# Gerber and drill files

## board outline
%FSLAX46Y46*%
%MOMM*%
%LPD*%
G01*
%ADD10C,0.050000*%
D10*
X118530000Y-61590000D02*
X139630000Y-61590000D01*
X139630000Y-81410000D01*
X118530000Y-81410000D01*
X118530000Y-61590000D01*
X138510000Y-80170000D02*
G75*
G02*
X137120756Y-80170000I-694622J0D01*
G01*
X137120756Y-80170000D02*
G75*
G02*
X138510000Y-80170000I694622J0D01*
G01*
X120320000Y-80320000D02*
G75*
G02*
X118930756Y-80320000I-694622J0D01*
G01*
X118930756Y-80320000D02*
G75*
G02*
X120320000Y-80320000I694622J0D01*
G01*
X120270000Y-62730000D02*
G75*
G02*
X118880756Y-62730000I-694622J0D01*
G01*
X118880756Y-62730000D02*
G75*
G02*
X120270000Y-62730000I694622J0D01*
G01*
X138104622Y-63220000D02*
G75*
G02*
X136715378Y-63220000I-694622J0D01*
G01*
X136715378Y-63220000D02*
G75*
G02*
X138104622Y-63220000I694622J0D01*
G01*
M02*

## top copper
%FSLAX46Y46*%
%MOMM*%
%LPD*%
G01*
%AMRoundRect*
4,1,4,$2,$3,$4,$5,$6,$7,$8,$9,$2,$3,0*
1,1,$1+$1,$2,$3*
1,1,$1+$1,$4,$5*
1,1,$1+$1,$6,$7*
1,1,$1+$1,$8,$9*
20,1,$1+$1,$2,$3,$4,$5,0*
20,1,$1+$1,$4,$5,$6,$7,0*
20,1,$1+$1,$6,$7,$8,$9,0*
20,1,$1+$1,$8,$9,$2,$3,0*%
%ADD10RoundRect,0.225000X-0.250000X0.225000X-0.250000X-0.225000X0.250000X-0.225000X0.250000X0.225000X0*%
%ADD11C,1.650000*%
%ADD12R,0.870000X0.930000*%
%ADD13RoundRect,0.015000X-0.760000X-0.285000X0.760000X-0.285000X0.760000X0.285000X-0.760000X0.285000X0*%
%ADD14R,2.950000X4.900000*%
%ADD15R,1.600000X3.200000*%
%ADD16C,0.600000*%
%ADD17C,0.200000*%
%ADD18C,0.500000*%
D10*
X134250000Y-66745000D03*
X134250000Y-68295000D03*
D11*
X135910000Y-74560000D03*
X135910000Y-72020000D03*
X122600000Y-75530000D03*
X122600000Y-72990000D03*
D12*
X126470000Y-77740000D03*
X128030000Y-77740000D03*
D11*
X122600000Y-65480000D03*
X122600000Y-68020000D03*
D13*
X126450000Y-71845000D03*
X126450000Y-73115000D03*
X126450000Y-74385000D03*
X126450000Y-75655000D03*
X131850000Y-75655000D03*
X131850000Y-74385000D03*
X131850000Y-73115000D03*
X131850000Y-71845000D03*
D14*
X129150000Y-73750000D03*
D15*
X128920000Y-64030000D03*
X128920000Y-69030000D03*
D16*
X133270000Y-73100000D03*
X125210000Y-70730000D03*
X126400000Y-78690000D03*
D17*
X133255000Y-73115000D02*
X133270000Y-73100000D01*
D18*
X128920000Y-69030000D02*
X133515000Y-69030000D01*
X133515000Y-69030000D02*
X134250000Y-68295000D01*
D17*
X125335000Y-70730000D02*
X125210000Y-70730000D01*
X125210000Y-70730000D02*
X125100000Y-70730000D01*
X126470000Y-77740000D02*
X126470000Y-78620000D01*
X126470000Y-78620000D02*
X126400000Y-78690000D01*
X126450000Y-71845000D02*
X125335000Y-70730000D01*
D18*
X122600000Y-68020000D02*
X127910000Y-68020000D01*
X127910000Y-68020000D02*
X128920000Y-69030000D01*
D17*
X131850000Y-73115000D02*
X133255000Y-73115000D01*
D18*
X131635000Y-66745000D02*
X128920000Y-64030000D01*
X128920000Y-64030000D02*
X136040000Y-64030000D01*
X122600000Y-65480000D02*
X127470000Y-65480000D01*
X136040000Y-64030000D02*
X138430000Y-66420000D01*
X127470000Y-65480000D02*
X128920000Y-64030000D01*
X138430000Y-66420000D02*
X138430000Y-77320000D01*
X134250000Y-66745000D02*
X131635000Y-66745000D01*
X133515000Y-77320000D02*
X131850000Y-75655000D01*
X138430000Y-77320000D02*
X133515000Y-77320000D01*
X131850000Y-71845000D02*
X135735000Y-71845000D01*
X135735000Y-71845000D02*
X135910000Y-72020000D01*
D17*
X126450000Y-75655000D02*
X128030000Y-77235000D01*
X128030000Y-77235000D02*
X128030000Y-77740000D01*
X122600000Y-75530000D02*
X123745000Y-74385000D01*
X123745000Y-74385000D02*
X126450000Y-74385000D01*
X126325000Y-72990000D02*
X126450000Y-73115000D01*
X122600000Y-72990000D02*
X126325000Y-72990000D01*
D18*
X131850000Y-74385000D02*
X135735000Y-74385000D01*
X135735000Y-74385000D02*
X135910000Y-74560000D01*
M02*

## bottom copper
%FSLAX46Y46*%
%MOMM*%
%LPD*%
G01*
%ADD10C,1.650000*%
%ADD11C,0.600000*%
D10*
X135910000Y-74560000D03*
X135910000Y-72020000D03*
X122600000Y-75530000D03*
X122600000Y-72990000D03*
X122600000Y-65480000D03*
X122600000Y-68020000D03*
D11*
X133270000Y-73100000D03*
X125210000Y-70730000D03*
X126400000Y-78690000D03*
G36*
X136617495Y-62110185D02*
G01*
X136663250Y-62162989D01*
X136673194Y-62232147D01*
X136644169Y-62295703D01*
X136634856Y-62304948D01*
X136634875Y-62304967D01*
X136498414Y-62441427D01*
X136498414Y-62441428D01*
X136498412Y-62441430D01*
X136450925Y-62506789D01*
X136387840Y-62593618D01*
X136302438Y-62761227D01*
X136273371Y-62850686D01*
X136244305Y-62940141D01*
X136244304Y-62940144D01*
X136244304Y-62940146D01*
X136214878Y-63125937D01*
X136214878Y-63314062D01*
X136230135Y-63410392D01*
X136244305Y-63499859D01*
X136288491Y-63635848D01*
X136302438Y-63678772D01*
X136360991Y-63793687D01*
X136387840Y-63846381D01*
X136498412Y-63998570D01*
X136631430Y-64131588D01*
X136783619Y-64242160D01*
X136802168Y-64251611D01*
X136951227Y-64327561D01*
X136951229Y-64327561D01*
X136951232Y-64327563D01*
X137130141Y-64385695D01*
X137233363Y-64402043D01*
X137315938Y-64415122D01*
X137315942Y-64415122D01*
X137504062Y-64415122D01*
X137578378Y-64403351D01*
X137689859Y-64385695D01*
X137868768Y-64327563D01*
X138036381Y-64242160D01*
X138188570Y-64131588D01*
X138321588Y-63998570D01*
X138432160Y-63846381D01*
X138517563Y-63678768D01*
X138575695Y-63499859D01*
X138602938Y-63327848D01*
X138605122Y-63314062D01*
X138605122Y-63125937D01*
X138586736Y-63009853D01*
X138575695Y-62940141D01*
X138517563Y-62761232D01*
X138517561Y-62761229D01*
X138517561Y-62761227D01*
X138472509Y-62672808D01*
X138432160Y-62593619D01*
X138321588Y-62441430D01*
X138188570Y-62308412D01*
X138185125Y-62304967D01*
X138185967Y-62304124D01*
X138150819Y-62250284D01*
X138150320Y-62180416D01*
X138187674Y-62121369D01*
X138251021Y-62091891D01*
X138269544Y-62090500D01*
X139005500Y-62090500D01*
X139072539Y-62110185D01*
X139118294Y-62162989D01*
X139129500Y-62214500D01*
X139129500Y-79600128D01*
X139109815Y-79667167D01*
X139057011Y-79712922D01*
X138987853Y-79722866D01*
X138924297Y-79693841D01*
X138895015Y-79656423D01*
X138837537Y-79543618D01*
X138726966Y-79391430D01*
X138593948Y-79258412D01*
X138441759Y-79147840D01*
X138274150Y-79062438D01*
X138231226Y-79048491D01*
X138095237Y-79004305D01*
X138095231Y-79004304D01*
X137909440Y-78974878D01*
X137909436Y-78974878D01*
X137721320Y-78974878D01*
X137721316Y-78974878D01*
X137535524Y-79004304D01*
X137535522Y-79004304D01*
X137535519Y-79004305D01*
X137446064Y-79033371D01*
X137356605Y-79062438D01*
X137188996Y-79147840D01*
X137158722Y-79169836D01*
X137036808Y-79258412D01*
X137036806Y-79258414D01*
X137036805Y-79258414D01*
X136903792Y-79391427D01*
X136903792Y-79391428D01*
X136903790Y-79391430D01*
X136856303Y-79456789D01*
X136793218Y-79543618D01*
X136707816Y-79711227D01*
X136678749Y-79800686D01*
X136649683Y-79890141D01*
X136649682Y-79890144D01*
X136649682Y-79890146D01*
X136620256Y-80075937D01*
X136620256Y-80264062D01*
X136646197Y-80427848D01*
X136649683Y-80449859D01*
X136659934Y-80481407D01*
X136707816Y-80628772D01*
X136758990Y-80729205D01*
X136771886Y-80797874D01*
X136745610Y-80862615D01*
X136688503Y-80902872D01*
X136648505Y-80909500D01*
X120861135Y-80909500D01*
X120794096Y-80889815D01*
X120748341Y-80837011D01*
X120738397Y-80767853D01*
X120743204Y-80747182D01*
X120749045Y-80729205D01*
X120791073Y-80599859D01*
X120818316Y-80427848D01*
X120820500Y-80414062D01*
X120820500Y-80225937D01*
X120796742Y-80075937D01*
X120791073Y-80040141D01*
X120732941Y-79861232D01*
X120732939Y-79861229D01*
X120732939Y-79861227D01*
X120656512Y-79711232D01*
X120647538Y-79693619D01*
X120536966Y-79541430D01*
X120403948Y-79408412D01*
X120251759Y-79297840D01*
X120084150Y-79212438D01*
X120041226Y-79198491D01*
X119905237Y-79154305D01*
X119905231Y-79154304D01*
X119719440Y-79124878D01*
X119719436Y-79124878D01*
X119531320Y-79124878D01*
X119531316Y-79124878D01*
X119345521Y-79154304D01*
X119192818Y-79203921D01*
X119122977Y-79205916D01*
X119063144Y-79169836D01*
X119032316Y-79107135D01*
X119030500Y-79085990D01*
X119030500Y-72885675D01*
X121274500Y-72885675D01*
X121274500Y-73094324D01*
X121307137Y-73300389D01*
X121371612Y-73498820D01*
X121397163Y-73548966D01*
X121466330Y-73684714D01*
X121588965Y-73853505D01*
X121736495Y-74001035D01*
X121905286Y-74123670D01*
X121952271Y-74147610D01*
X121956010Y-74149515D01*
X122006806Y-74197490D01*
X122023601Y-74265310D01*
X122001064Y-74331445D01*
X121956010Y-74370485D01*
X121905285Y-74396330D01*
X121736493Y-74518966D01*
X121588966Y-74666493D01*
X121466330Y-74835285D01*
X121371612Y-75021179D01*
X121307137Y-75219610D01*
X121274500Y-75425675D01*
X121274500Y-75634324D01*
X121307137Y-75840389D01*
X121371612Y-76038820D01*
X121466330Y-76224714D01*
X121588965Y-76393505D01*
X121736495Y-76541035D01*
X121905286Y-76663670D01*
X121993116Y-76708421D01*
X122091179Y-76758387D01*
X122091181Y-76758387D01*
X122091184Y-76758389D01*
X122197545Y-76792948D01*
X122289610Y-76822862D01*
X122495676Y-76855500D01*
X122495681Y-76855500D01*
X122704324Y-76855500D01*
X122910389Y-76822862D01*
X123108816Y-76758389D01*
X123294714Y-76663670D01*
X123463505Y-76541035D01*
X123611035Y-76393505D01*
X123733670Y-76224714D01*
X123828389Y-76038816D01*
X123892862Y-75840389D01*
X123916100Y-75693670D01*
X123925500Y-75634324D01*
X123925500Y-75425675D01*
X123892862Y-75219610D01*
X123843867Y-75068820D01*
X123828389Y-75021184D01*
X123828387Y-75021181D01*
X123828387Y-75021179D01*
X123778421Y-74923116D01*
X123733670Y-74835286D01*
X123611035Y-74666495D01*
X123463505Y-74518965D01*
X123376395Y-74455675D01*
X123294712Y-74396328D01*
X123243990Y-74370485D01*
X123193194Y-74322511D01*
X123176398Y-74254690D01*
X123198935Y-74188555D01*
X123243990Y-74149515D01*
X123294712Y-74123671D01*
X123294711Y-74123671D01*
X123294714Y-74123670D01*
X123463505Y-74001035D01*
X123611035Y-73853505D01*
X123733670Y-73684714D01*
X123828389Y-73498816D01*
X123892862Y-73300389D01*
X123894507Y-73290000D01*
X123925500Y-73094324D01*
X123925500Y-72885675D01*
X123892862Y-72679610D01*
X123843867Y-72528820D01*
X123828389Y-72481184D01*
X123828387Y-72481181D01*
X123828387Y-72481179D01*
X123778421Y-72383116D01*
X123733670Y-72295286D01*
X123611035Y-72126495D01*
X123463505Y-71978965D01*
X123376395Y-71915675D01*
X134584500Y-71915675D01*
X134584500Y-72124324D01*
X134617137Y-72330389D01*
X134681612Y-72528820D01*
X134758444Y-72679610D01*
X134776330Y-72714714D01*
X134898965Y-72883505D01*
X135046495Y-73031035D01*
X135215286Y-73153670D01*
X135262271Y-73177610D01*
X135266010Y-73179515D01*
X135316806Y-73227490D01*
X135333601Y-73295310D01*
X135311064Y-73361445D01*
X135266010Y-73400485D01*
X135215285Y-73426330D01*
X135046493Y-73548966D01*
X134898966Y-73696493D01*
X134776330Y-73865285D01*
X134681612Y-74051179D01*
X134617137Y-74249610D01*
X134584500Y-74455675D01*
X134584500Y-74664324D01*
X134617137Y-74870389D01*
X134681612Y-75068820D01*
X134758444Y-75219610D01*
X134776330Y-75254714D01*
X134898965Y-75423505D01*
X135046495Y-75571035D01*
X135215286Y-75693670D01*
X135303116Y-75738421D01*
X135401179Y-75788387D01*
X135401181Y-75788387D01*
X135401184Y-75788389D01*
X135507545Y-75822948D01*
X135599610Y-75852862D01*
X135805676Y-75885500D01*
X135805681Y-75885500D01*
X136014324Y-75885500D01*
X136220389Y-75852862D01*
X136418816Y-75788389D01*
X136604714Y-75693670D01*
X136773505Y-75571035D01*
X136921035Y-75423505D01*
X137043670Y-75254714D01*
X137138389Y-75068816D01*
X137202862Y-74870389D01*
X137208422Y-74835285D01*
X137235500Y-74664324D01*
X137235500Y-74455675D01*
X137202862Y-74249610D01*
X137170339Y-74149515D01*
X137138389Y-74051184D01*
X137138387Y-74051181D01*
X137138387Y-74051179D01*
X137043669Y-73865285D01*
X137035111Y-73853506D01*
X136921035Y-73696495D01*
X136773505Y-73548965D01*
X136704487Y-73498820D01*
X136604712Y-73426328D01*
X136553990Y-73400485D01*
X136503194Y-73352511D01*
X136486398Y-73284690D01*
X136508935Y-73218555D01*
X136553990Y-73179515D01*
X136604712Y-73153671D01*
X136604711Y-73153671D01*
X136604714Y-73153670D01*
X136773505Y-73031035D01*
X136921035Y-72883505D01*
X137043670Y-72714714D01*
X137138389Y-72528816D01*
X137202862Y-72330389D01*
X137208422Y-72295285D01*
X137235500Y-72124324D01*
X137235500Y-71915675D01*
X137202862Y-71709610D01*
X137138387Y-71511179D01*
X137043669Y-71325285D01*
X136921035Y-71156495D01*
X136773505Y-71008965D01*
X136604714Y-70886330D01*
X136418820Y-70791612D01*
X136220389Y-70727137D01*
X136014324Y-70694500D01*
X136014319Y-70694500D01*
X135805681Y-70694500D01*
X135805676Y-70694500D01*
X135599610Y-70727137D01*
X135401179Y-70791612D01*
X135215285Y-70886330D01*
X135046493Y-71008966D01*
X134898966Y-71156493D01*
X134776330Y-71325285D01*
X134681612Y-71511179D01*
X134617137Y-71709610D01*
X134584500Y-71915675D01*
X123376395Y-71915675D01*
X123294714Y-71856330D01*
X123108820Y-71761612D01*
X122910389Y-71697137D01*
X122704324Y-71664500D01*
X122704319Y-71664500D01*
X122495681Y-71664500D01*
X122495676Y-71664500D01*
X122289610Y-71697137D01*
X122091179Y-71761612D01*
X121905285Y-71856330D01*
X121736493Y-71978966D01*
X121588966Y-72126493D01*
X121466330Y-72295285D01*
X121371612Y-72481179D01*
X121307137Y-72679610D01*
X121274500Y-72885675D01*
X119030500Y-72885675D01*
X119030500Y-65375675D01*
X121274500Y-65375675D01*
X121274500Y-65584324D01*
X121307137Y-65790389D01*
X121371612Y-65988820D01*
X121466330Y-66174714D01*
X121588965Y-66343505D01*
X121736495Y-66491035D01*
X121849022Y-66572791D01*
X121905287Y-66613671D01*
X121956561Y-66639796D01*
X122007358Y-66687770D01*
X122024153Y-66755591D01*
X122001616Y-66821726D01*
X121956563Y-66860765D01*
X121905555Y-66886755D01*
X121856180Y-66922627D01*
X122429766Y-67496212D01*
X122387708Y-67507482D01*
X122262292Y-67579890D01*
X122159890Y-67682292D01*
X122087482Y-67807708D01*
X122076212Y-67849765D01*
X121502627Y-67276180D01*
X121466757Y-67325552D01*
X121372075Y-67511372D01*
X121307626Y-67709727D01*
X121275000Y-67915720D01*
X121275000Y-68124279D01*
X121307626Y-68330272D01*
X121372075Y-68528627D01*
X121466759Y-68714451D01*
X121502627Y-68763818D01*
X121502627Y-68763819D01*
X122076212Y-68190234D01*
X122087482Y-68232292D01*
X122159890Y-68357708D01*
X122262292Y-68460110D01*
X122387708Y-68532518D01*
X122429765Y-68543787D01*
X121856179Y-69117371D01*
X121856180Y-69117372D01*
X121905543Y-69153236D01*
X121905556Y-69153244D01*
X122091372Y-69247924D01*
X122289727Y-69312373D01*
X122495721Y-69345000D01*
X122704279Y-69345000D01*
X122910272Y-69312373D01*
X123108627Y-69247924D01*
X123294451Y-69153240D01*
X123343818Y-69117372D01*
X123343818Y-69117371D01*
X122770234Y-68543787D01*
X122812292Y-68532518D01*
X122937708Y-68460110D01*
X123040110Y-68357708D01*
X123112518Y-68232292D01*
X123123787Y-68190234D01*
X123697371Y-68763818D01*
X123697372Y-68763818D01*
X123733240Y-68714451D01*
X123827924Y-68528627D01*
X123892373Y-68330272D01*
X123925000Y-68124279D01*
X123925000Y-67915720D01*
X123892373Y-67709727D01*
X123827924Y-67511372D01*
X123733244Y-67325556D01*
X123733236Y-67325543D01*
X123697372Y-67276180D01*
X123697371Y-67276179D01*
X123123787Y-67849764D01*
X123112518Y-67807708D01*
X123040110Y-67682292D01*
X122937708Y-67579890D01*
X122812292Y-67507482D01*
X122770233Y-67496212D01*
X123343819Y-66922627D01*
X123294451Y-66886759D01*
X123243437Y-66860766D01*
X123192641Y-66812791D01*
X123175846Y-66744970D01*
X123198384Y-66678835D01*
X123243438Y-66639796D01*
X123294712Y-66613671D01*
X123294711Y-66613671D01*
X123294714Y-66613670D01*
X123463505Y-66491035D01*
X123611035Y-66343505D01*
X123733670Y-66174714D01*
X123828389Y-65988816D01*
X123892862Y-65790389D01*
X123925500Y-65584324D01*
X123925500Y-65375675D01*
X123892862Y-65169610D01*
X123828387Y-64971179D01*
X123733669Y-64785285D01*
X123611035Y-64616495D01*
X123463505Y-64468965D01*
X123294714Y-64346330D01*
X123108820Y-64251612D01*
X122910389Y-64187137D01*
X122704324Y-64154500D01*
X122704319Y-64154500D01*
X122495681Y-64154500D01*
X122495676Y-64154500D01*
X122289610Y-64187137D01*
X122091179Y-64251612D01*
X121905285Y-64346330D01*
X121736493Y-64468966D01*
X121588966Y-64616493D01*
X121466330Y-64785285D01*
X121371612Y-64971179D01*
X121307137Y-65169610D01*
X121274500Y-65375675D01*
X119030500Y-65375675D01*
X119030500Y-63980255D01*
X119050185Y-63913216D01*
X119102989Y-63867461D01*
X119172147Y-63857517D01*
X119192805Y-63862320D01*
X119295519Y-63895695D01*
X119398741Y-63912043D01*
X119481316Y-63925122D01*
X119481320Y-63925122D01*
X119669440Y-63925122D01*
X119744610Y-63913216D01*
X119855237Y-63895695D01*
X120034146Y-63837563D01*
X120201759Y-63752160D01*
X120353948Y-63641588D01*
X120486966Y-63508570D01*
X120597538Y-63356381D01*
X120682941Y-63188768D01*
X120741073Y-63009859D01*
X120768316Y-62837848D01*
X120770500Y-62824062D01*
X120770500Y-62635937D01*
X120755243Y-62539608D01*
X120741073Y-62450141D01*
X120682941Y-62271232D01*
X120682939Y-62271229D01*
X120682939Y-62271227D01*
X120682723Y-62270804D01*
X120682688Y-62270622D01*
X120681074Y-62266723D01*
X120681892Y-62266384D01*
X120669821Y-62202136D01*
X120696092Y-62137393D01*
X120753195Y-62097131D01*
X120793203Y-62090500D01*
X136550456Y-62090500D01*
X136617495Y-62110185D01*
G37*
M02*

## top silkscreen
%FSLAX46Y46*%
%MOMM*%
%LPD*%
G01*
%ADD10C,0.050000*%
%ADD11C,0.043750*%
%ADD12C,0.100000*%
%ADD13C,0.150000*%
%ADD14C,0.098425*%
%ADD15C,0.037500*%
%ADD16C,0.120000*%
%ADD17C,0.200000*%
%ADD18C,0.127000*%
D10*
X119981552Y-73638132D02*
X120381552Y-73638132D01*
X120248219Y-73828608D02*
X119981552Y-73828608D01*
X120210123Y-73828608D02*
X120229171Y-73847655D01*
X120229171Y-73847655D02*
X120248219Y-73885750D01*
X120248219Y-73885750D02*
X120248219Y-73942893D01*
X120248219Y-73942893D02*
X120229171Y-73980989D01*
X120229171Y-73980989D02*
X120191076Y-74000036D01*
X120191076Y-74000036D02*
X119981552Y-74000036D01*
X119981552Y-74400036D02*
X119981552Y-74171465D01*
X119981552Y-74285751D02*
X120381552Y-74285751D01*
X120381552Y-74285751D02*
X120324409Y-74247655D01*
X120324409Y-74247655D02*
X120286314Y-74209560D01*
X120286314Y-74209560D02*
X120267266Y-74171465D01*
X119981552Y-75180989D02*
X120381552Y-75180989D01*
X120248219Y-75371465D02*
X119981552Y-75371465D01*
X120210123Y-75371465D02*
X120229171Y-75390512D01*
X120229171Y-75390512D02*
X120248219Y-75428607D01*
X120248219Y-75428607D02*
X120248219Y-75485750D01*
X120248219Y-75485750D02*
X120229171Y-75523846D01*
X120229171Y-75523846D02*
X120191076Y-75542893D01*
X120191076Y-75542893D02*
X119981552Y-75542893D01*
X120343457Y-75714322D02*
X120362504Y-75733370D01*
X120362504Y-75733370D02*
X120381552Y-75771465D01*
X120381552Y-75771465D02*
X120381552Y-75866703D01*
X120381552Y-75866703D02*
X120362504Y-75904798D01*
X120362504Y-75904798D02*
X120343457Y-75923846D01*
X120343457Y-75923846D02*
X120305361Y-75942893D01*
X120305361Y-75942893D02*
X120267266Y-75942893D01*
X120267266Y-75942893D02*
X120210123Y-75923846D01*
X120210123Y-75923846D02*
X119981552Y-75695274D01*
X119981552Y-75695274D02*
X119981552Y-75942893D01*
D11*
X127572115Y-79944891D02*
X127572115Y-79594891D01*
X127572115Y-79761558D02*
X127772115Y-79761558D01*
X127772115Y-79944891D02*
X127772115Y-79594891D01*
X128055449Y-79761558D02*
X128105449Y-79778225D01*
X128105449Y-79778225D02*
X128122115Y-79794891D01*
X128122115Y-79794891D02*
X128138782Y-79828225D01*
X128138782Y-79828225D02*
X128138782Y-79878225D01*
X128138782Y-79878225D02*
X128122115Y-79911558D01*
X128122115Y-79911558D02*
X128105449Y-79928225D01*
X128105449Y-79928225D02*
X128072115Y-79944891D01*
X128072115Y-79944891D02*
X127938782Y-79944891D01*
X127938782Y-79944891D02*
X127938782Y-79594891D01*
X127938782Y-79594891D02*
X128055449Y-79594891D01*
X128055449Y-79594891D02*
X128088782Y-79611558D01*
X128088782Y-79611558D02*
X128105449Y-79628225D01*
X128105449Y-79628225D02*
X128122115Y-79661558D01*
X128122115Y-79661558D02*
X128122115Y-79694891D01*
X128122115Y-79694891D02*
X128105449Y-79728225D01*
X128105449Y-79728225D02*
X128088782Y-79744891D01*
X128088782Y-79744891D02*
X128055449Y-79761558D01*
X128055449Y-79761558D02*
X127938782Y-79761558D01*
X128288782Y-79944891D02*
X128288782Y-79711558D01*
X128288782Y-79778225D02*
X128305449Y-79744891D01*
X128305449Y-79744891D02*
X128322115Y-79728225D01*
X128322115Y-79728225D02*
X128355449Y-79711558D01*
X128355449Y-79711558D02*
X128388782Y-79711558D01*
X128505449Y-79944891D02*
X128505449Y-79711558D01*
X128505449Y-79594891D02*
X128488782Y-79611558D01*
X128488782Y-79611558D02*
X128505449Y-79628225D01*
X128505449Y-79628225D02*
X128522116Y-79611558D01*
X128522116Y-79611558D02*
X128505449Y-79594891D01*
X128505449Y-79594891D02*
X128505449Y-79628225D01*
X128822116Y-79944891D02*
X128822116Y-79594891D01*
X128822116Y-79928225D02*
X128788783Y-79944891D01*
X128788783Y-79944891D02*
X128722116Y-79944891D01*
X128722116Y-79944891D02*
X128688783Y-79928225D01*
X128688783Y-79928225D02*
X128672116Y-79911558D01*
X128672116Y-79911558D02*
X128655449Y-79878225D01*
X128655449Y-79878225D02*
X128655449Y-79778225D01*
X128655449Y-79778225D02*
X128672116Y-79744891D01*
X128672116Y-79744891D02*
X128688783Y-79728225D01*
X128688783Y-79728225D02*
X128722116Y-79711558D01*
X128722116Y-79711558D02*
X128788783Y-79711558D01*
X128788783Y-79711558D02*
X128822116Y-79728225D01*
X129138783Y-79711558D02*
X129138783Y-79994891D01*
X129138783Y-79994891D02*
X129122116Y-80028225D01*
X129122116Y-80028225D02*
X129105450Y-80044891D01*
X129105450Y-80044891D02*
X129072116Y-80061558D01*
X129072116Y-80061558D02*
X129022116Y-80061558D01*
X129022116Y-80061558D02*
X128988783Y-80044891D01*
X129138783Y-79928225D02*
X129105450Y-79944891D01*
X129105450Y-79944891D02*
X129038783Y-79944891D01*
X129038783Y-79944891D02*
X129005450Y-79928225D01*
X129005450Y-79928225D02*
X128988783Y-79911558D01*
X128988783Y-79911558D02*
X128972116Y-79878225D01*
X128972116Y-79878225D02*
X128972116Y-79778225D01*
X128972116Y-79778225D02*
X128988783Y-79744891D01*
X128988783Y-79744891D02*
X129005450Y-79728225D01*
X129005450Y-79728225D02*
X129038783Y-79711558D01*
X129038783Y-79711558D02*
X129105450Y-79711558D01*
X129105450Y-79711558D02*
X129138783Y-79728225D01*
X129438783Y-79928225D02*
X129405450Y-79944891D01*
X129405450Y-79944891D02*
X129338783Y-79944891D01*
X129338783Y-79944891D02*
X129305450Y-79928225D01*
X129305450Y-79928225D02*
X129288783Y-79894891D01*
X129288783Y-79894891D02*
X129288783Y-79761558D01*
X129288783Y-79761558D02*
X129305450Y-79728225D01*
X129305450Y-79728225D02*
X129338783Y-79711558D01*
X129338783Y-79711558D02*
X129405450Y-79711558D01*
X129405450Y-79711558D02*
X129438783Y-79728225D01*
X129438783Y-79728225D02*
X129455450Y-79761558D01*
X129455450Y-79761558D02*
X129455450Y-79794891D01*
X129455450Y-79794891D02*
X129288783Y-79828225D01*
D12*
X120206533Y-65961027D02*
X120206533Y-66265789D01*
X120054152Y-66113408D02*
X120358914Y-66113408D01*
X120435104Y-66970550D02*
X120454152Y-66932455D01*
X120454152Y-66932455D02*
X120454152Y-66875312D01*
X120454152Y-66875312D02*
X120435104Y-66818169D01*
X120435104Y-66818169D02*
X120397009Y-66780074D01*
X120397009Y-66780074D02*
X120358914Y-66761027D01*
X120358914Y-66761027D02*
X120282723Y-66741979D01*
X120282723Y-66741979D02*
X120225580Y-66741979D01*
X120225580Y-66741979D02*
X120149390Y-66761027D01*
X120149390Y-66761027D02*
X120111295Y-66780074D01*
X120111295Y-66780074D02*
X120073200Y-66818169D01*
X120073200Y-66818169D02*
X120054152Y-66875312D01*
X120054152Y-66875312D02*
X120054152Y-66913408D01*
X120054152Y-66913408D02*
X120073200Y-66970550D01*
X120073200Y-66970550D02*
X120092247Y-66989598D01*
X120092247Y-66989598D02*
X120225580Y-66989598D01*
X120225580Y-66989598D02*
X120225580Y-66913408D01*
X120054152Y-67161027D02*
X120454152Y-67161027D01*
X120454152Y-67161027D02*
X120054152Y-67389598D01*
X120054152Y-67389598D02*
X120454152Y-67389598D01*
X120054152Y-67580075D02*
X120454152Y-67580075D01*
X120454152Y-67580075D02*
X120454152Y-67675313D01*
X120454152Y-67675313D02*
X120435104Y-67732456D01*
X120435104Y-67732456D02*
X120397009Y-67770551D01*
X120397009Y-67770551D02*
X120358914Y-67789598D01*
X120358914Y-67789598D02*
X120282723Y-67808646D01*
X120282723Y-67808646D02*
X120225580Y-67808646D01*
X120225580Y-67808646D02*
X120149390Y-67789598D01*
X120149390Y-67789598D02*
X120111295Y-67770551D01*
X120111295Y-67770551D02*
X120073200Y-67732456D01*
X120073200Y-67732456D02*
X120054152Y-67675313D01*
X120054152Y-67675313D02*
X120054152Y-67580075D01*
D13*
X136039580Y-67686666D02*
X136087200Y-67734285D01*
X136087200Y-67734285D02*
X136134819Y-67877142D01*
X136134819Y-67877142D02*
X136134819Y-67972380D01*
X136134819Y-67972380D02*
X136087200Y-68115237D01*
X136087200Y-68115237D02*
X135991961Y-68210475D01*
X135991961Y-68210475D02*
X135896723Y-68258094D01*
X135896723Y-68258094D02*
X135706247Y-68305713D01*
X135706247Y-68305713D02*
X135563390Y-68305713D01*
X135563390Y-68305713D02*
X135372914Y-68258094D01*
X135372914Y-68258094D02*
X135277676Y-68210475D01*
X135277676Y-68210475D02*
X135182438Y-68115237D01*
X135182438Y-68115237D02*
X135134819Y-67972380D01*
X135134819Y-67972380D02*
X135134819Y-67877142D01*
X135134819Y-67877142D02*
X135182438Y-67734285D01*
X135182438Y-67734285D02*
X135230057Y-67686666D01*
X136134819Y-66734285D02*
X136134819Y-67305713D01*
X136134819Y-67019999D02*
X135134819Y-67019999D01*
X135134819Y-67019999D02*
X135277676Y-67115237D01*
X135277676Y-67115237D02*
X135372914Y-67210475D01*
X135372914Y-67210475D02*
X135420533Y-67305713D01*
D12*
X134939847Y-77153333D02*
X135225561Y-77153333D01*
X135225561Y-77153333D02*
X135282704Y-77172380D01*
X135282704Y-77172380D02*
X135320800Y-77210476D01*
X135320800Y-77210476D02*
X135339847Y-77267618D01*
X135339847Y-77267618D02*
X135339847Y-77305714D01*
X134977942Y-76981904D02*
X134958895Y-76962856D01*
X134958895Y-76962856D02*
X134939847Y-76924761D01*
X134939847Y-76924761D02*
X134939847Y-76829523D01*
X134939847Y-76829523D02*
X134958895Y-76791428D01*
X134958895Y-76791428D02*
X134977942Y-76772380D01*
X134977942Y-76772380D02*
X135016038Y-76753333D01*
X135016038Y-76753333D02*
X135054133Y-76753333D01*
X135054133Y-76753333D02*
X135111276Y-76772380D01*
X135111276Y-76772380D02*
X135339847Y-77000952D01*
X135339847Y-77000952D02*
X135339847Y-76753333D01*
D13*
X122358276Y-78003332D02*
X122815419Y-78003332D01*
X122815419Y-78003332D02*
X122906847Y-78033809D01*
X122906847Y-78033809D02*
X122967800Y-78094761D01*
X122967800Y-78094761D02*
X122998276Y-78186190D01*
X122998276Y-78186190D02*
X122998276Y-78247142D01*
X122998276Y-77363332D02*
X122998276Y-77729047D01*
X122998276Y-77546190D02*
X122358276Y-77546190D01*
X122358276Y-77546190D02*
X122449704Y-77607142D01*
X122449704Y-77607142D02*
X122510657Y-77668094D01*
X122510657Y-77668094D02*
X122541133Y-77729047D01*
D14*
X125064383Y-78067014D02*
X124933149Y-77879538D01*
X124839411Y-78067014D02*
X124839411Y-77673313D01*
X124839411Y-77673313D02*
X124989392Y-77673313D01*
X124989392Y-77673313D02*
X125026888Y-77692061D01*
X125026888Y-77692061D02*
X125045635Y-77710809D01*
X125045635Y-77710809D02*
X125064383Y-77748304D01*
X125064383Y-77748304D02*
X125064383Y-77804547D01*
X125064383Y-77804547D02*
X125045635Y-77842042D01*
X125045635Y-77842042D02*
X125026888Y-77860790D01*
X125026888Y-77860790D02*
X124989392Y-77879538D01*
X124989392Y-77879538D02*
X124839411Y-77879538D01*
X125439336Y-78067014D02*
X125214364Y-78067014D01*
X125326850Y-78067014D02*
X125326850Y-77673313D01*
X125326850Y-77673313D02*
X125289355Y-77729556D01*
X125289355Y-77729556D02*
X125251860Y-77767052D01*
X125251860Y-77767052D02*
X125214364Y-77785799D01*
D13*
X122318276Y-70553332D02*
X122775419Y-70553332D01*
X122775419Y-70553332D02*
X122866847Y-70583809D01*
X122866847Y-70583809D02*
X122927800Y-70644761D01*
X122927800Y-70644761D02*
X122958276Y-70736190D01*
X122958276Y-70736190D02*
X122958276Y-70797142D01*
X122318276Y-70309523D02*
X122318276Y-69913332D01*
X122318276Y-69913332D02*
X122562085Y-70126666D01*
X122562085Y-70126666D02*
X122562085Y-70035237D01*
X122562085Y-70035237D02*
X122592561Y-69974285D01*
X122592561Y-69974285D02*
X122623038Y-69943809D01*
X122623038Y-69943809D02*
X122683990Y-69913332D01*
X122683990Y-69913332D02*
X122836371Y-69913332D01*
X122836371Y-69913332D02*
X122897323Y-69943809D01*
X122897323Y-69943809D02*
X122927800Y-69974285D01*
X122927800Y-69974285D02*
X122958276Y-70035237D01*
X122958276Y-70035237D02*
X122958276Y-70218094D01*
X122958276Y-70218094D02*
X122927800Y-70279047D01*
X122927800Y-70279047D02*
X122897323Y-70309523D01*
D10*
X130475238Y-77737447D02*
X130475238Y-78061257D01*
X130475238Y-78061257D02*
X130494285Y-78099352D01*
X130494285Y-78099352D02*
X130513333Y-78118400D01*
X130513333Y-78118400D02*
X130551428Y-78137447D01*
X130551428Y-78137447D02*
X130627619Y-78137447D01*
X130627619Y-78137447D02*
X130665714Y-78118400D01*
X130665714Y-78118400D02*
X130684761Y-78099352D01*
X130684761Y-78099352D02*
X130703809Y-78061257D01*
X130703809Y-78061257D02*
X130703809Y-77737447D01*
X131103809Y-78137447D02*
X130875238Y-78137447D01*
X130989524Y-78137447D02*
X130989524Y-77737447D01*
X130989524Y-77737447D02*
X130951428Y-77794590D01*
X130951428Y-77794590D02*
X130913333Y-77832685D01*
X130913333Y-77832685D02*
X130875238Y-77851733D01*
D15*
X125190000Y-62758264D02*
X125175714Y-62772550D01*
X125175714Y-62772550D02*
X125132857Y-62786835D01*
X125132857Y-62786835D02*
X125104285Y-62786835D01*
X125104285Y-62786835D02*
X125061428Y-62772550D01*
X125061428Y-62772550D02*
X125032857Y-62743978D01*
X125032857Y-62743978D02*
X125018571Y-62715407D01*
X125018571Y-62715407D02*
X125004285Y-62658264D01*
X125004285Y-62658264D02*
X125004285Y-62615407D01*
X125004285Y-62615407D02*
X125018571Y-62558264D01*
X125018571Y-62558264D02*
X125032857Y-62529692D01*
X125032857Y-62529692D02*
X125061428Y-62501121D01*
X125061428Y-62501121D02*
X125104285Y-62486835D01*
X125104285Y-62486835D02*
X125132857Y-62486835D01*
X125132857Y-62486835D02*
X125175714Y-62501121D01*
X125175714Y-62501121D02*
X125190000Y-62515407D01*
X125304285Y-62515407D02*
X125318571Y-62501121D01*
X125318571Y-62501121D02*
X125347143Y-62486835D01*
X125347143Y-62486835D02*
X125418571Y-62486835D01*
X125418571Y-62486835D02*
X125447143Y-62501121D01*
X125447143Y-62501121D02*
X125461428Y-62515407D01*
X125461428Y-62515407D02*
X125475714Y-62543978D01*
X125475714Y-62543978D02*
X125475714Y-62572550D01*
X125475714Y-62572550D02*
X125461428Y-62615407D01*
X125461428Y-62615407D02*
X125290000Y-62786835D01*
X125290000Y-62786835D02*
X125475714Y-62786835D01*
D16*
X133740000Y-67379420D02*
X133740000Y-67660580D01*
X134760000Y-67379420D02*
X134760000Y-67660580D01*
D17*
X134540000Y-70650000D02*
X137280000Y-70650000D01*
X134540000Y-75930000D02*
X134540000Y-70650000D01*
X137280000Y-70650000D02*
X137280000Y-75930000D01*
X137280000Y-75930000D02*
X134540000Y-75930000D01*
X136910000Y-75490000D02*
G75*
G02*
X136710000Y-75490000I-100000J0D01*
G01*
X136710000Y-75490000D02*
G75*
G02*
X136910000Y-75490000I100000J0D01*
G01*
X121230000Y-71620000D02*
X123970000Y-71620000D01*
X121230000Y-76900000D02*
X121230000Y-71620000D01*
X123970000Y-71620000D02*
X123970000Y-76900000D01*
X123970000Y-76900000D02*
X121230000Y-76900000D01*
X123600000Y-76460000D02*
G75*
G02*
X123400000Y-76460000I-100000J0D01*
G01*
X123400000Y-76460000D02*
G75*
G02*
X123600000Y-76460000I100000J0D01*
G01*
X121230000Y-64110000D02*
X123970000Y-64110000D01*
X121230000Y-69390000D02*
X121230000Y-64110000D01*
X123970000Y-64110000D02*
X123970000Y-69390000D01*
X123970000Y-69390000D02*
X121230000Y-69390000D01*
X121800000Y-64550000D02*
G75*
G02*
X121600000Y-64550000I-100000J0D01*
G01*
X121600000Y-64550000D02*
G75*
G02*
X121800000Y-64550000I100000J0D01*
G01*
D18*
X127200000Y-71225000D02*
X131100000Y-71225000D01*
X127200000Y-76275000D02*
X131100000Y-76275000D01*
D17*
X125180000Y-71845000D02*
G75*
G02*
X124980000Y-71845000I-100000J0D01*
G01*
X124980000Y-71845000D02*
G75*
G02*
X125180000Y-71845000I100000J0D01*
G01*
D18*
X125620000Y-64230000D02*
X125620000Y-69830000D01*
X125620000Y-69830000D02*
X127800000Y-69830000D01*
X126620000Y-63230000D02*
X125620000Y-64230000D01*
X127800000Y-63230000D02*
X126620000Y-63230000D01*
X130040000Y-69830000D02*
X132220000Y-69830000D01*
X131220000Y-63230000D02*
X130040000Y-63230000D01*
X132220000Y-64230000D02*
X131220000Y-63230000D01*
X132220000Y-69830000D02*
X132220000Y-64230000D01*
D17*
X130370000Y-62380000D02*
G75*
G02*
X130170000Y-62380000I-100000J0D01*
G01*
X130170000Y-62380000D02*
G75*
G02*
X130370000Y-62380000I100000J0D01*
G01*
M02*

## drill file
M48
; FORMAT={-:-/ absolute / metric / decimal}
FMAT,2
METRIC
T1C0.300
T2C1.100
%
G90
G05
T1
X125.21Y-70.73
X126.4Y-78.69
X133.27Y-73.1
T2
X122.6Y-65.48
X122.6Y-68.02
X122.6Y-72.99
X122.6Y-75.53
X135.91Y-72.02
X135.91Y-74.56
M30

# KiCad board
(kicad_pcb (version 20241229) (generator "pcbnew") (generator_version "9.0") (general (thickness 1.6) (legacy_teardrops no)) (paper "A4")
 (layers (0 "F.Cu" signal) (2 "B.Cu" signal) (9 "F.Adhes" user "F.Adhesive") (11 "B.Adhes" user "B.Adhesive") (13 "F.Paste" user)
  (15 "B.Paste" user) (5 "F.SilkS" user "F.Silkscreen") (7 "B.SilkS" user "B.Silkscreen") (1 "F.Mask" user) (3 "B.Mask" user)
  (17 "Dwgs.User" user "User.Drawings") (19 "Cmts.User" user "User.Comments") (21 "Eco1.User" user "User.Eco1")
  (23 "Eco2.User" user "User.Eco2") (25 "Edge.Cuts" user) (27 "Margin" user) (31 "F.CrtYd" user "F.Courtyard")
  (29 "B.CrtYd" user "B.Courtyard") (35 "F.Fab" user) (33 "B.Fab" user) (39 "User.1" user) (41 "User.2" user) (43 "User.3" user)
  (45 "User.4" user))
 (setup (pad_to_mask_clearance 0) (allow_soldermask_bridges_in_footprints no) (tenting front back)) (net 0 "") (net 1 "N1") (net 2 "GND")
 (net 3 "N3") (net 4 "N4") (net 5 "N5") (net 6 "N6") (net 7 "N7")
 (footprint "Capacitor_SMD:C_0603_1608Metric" (layer "F.Cu") (at 134.25 67.52 -90)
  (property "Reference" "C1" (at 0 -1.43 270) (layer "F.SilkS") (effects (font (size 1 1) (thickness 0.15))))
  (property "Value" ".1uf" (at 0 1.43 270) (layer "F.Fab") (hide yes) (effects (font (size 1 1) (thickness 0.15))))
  (fp_line (start -0.14058 0.51) (end 0.14058 0.51) (stroke (width 0.12) (type solid)) (layer "F.SilkS"))
  (fp_line (start -0.14058 -0.51) (end 0.14058 -0.51) (stroke (width 0.12) (type solid)) (layer "F.SilkS"))
  (pad "1" smd roundrect (at -0.775 0 270) (size 0.9 0.95) (layers "F.Cu" "F.Mask" "F.Paste") (roundrect_rratio 0.25) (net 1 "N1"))
  (pad "2" smd roundrect (at 0.775 0 270) (size 0.9 0.95) (layers "F.Cu" "F.Mask" "F.Paste") (roundrect_rratio 0.25) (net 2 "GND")))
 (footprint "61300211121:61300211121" (layer "F.Cu") (at 135.91 73.29 90)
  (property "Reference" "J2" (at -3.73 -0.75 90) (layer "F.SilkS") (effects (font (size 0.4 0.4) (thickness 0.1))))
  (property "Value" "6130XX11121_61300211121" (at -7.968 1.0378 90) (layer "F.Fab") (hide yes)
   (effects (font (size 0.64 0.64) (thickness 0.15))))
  (fp_line (start 2.64 -1.37) (end 2.64 1.37) (stroke (width 0.2) (type solid)) (layer "F.SilkS"))
  (fp_line (start -2.64 -1.37) (end 2.64 -1.37) (stroke (width 0.2) (type solid)) (layer "F.SilkS"))
  (fp_line (start 2.64 1.37) (end -2.64 1.37) (stroke (width 0.2) (type solid)) (layer "F.SilkS"))
  (fp_line (start -2.64 1.37) (end -2.64 -1.37) (stroke (width 0.2) (type solid)) (layer "F.SilkS"))
  (fp_circle (center -2.2 0.9) (end -2.1 0.9) (stroke (width 0.2) (type solid)) (fill no) (layer "F.SilkS"))
  (pad "1" thru_hole circle (at -1.27 0 90) (size 1.65 1.65) (drill 1.1) (layers "*.Cu" "*.Mask") (remove_unused_layers no) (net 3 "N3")
   (solder_mask_margin 0.102))
  (pad "2" thru_hole circle (at 1.27 0 90) (size 1.65 1.65) (drill 1.1) (layers "*.Cu" "*.Mask") (remove_unused_layers no) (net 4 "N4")
   (solder_mask_margin 0.102)))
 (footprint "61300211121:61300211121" (layer "F.Cu") (at 122.6 74.26 90)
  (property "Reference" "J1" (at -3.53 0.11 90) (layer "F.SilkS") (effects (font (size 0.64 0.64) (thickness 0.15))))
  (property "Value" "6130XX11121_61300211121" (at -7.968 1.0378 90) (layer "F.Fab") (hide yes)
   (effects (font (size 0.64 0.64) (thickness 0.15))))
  (fp_line (start 2.64 -1.37) (end 2.64 1.37) (stroke (width 0.2) (type solid)) (layer "F.SilkS"))
  (fp_line (start -2.64 -1.37) (end 2.64 -1.37) (stroke (width 0.2) (type solid)) (layer "F.SilkS"))
  (fp_line (start 2.64 1.37) (end -2.64 1.37) (stroke (width 0.2) (type solid)) (layer "F.SilkS"))
  (fp_line (start -2.64 1.37) (end -2.64 -1.37) (stroke (width 0.2) (type solid)) (layer "F.SilkS"))
  (fp_circle (center -2.2 0.9) (end -2.1 0.9) (stroke (width 0.2) (type solid)) (fill no) (layer "F.SilkS"))
  (pad "1" thru_hole circle (at -1.27 0 90) (size 1.65 1.65) (drill 1.1) (layers "*.Cu" "*.Mask") (remove_unused_layers no) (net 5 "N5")
   (solder_mask_margin 0.102))
  (pad "2" thru_hole circle (at 1.27 0 90) (size 1.65 1.65) (drill 1.1) (layers "*.Cu" "*.Mask") (remove_unused_layers no) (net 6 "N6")
   (solder_mask_margin 0.102)))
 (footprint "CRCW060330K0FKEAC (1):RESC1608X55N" (layer "F.Cu") (at 127.25 77.74)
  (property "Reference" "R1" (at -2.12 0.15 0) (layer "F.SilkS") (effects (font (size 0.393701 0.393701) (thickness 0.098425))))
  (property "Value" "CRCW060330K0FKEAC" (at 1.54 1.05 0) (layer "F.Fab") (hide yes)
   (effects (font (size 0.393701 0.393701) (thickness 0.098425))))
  (pad "1" smd rect (at -0.78 0) (size 0.87 0.93) (layers "F.Cu" "F.Mask" "F.Paste") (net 2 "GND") (solder_mask_margin 0.102))
  (pad "2" smd rect (at 0.78 0) (size 0.87 0.93) (layers "F.Cu" "F.Mask" "F.Paste") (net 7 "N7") (solder_mask_margin 0.102)))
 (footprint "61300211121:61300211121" (layer "F.Cu") (at 122.6 66.75 -90)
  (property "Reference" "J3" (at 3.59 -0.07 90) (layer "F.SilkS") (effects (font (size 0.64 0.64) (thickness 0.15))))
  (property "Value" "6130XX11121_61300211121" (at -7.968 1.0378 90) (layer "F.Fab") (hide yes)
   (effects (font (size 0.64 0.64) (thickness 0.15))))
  (fp_line (start -2.64 1.37) (end -2.64 -1.37) (stroke (width 0.2) (type solid)) (layer "F.SilkS"))
  (fp_line (start 2.64 1.37) (end -2.64 1.37) (stroke (width 0.2) (type solid)) (layer "F.SilkS"))
  (fp_line (start -2.64 -1.37) (end 2.64 -1.37) (stroke (width 0.2) (type solid)) (layer "F.SilkS"))
  (fp_line (start 2.64 -1.37) (end 2.64 1.37) (stroke (width 0.2) (type solid)) (layer "F.SilkS"))
  (fp_circle (center -2.2 0.9) (end -2.1 0.9) (stroke (width 0.2) (type solid)) (fill no) (layer "F.SilkS"))
  (pad "1" thru_hole circle (at -1.27 0 270) (size 1.65 1.65) (drill 1.1) (layers "*.Cu" "*.Mask") (remove_unused_layers no) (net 1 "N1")
   (solder_mask_margin 0.102))
  (pad "2" thru_hole circle (at 1.27 0 270) (size 1.65 1.65) (drill 1.1) (layers "*.Cu" "*.Mask") (remove_unused_layers no) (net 2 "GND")
   (solder_mask_margin 0.102)))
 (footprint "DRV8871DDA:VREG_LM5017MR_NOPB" (layer "F.Cu") (at 129.15 73.75)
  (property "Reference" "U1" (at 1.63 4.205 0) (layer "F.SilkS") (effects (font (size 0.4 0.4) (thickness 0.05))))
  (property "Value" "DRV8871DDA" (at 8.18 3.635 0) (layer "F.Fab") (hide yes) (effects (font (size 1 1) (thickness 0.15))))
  (fp_line (start -1.95 -2.525) (end 1.95 -2.525) (stroke (width 0.127) (type solid)) (layer "F.SilkS"))
  (fp_line (start -1.95 2.525) (end 1.95 2.525) (stroke (width 0.127) (type solid)) (layer "F.SilkS"))
  (fp_circle (center -4.07 -1.905) (end -3.97 -1.905) (stroke (width 0.2) (type solid)) (fill no) (layer "F.SilkS"))
  (pad "1" smd roundrect (at -2.7 -1.905) (size 1.55 0.6) (layers "F.Cu" "F.Paste") (roundrect_rratio 0.025) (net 2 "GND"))
  (pad "2" smd roundrect (at -2.7 -0.635) (size 1.55 0.6) (layers "F.Cu" "F.Paste") (roundrect_rratio 0.025) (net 6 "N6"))
  (pad "3" smd roundrect (at -2.7 0.635) (size 1.55 0.6) (layers "F.Cu" "F.Paste") (roundrect_rratio 0.025) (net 5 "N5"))
  (pad "4" smd roundrect (at -2.7 1.905) (size 1.55 0.6) (layers "F.Cu" "F.Paste") (roundrect_rratio 0.025) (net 7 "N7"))
  (pad "5" smd roundrect (at 2.7 1.905) (size 1.55 0.6) (layers "F.Cu" "F.Paste") (roundrect_rratio 0.025) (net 1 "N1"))
  (pad "6" smd roundrect (at 2.7 0.635) (size 1.55 0.6) (layers "F.Cu" "F.Paste") (roundrect_rratio 0.025) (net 3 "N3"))
  (pad "7" smd roundrect (at 2.7 -0.635) (size 1.55 0.6) (layers "F.Cu" "F.Paste") (roundrect_rratio 0.025) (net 2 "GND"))
  (pad "8" smd roundrect (at 2.7 -1.905) (size 1.55 0.6) (layers "F.Cu" "F.Paste") (roundrect_rratio 0.025) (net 4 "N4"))
  (pad "9" smd rect (at 0 0) (size 2.95 4.9) (layers "F.Cu")))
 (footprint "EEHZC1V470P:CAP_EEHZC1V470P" (layer "F.Cu") (at 128.92 66.53 -90)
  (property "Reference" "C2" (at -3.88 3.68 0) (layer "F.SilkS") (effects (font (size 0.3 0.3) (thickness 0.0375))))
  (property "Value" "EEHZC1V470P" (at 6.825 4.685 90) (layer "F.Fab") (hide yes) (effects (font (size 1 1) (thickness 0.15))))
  (fp_line (start -2.3 3.3) (end 3.3 3.3) (stroke (width 0.127) (type solid)) (layer "F.SilkS"))
  (fp_line (start 3.3 3.3) (end 3.3 1.12) (stroke (width 0.127) (type solid)) (layer "F.SilkS"))
  (fp_line (start -3.3 2.3) (end -2.3 3.3) (stroke (width 0.127) (type solid)) (layer "F.SilkS"))
  (fp_line (start -3.3 1.12) (end -3.3 2.3) (stroke (width 0.127) (type solid)) (layer "F.SilkS"))
  (fp_line (start 3.3 -1.12) (end 3.3 -3.3) (stroke (width 0.127) (type solid)) (layer "F.SilkS"))
  (fp_line (start -3.3 -2.3) (end -3.3 -1.12) (stroke (width 0.127) (type solid)) (layer "F.SilkS"))
  (fp_line (start -2.3 -3.3) (end -3.3 -2.3) (stroke (width 0.127) (type solid)) (layer "F.SilkS"))
  (fp_line (start 3.3 -3.3) (end -2.3 -3.3) (stroke (width 0.127) (type solid)) (layer "F.SilkS"))
  (fp_circle (center -4.15 -1.35) (end -4.05 -1.35) (stroke (width 0.2) (type solid)) (fill no) (layer "F.SilkS"))
  (pad "1" smd rect (at -2.5 0 270) (size 3.2 1.6) (layers "F.Cu" "F.Mask" "F.Paste") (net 1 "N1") (solder_mask_margin 0.102))
  (pad "2" smd rect (at 2.5 0 270) (size 3.2 1.6) (layers "F.Cu" "F.Mask" "F.Paste") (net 2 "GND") (solder_mask_margin 0.102)))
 (gr_rect (start 118.53 61.59) (end 139.63 81.41) (stroke (width 0.05) (type default)) (fill no) (layer "Edge.Cuts"))
 (gr_circle (center 137.815378 80.17) (end 138.165378 80.77) (stroke (width 0.05) (type default)) (fill no) (layer "Edge.Cuts"))
 (gr_circle (center 119.625378 80.32) (end 119.975378 80.92) (stroke (width 0.05) (type default)) (fill no) (layer "Edge.Cuts"))
 (gr_circle (center 119.575378 62.73) (end 119.925378 63.33) (stroke (width 0.05) (type default)) (fill no) (layer "Edge.Cuts"))
 (gr_circle (center 137.41 63.22) (end 137.76 63.82) (stroke (width 0.05) (type default)) (fill no) (layer "Edge.Cuts"))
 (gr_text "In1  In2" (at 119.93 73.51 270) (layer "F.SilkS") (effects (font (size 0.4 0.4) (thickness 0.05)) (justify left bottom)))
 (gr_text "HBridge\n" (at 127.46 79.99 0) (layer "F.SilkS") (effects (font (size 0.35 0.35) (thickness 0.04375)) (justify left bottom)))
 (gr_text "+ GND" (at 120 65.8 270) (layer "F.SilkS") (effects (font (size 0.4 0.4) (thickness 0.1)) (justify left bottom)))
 (segment (start 133.255 73.115) (end 133.27 73.1) (width 0.2) (layer "F.Cu") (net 2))
 (segment (start 128.92 69.03) (end 133.515 69.03) (width 0.5) (layer "F.Cu") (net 2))
 (segment (start 133.515 69.03) (end 134.25 68.295) (width 0.5) (layer "F.Cu") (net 2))
 (segment (start 125.335 70.73) (end 125.21 70.73) (width 0.2) (layer "F.Cu") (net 2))
 (segment (start 125.21 70.73) (end 125.1 70.73) (width 0.2) (layer "F.Cu") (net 2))
 (segment (start 126.47 77.74) (end 126.47 78.62) (width 0.2) (layer "F.Cu") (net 2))
 (segment (start 126.47 78.62) (end 126.4 78.69) (width 0.2) (layer "F.Cu") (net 2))
 (segment (start 126.45 71.845) (end 125.335 70.73) (width 0.2) (layer "F.Cu") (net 2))
 (segment (start 122.6 68.02) (end 127.91 68.02) (width 0.5) (layer "F.Cu") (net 2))
 (segment (start 127.91 68.02) (end 128.92 69.03) (width 0.5) (layer "F.Cu") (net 2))
 (segment (start 131.85 73.115) (end 133.255 73.115) (width 0.2) (layer "F.Cu") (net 2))
 (via (at 133.27 73.1) (size 0.6) (drill 0.3) (layers "F.Cu" "B.Cu") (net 2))
 (via (at 125.21 70.73) (size 0.6) (drill 0.3) (layers "F.Cu" "B.Cu") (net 2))
 (via (at 126.4 78.69) (size 0.6) (drill 0.3) (layers "F.Cu" "B.Cu") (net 2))
 (segment (start 131.635 66.745) (end 128.92 64.03) (width 0.5) (layer "F.Cu") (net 1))
 (segment (start 128.92 64.03) (end 136.04 64.03) (width 0.5) (layer "F.Cu") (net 1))
 (segment (start 122.6 65.48) (end 127.47 65.48) (width 0.5) (layer "F.Cu") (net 1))
 (segment (start 136.04 64.03) (end 138.43 66.42) (width 0.5) (layer "F.Cu") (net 1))
 (segment (start 127.47 65.48) (end 128.92 64.03) (width 0.5) (layer "F.Cu") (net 1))
 (segment (start 138.43 66.42) (end 138.43 77.32) (width 0.5) (layer "F.Cu") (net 1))
 (segment (start 134.25 66.745) (end 131.635 66.745) (width 0.5) (layer "F.Cu") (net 1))
 (segment (start 133.515 77.32) (end 131.85 75.655) (width 0.5) (layer "F.Cu") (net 1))
 (segment (start 138.43 77.32) (end 133.515 77.32) (width 0.5) (layer "F.Cu") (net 1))
 (segment (start 131.85 71.845) (end 135.735 71.845) (width 0.5) (layer "F.Cu") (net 4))
 (segment (start 135.735 71.845) (end 135.91 72.02) (width 0.5) (layer "F.Cu") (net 4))
 (segment (start 126.45 75.655) (end 128.03 77.235) (width 0.2) (layer "F.Cu") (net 7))
 (segment (start 128.03 77.235) (end 128.03 77.74) (width 0.2) (layer "F.Cu") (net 7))
 (segment (start 122.6 75.53) (end 123.745 74.385) (width 0.2) (layer "F.Cu") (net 5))
 (segment (start 123.745 74.385) (end 126.45 74.385) (width 0.2) (layer "F.Cu") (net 5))
 (segment (start 126.325 72.99) (end 126.45 73.115) (width 0.2) (layer "F.Cu") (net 6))
 (segment (start 122.6 72.99) (end 126.325 72.99) (width 0.2) (layer "F.Cu") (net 6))
 (segment (start 131.85 74.385) (end 135.735 74.385) (width 0.5) (layer "F.Cu") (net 3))
 (segment (start 135.735 74.385) (end 135.91 74.56) (width 0.5) (layer "F.Cu") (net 3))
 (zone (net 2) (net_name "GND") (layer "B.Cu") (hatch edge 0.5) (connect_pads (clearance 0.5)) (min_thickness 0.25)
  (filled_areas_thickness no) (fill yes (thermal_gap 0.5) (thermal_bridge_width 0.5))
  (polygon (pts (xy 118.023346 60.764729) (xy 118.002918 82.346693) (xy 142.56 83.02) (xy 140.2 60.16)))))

